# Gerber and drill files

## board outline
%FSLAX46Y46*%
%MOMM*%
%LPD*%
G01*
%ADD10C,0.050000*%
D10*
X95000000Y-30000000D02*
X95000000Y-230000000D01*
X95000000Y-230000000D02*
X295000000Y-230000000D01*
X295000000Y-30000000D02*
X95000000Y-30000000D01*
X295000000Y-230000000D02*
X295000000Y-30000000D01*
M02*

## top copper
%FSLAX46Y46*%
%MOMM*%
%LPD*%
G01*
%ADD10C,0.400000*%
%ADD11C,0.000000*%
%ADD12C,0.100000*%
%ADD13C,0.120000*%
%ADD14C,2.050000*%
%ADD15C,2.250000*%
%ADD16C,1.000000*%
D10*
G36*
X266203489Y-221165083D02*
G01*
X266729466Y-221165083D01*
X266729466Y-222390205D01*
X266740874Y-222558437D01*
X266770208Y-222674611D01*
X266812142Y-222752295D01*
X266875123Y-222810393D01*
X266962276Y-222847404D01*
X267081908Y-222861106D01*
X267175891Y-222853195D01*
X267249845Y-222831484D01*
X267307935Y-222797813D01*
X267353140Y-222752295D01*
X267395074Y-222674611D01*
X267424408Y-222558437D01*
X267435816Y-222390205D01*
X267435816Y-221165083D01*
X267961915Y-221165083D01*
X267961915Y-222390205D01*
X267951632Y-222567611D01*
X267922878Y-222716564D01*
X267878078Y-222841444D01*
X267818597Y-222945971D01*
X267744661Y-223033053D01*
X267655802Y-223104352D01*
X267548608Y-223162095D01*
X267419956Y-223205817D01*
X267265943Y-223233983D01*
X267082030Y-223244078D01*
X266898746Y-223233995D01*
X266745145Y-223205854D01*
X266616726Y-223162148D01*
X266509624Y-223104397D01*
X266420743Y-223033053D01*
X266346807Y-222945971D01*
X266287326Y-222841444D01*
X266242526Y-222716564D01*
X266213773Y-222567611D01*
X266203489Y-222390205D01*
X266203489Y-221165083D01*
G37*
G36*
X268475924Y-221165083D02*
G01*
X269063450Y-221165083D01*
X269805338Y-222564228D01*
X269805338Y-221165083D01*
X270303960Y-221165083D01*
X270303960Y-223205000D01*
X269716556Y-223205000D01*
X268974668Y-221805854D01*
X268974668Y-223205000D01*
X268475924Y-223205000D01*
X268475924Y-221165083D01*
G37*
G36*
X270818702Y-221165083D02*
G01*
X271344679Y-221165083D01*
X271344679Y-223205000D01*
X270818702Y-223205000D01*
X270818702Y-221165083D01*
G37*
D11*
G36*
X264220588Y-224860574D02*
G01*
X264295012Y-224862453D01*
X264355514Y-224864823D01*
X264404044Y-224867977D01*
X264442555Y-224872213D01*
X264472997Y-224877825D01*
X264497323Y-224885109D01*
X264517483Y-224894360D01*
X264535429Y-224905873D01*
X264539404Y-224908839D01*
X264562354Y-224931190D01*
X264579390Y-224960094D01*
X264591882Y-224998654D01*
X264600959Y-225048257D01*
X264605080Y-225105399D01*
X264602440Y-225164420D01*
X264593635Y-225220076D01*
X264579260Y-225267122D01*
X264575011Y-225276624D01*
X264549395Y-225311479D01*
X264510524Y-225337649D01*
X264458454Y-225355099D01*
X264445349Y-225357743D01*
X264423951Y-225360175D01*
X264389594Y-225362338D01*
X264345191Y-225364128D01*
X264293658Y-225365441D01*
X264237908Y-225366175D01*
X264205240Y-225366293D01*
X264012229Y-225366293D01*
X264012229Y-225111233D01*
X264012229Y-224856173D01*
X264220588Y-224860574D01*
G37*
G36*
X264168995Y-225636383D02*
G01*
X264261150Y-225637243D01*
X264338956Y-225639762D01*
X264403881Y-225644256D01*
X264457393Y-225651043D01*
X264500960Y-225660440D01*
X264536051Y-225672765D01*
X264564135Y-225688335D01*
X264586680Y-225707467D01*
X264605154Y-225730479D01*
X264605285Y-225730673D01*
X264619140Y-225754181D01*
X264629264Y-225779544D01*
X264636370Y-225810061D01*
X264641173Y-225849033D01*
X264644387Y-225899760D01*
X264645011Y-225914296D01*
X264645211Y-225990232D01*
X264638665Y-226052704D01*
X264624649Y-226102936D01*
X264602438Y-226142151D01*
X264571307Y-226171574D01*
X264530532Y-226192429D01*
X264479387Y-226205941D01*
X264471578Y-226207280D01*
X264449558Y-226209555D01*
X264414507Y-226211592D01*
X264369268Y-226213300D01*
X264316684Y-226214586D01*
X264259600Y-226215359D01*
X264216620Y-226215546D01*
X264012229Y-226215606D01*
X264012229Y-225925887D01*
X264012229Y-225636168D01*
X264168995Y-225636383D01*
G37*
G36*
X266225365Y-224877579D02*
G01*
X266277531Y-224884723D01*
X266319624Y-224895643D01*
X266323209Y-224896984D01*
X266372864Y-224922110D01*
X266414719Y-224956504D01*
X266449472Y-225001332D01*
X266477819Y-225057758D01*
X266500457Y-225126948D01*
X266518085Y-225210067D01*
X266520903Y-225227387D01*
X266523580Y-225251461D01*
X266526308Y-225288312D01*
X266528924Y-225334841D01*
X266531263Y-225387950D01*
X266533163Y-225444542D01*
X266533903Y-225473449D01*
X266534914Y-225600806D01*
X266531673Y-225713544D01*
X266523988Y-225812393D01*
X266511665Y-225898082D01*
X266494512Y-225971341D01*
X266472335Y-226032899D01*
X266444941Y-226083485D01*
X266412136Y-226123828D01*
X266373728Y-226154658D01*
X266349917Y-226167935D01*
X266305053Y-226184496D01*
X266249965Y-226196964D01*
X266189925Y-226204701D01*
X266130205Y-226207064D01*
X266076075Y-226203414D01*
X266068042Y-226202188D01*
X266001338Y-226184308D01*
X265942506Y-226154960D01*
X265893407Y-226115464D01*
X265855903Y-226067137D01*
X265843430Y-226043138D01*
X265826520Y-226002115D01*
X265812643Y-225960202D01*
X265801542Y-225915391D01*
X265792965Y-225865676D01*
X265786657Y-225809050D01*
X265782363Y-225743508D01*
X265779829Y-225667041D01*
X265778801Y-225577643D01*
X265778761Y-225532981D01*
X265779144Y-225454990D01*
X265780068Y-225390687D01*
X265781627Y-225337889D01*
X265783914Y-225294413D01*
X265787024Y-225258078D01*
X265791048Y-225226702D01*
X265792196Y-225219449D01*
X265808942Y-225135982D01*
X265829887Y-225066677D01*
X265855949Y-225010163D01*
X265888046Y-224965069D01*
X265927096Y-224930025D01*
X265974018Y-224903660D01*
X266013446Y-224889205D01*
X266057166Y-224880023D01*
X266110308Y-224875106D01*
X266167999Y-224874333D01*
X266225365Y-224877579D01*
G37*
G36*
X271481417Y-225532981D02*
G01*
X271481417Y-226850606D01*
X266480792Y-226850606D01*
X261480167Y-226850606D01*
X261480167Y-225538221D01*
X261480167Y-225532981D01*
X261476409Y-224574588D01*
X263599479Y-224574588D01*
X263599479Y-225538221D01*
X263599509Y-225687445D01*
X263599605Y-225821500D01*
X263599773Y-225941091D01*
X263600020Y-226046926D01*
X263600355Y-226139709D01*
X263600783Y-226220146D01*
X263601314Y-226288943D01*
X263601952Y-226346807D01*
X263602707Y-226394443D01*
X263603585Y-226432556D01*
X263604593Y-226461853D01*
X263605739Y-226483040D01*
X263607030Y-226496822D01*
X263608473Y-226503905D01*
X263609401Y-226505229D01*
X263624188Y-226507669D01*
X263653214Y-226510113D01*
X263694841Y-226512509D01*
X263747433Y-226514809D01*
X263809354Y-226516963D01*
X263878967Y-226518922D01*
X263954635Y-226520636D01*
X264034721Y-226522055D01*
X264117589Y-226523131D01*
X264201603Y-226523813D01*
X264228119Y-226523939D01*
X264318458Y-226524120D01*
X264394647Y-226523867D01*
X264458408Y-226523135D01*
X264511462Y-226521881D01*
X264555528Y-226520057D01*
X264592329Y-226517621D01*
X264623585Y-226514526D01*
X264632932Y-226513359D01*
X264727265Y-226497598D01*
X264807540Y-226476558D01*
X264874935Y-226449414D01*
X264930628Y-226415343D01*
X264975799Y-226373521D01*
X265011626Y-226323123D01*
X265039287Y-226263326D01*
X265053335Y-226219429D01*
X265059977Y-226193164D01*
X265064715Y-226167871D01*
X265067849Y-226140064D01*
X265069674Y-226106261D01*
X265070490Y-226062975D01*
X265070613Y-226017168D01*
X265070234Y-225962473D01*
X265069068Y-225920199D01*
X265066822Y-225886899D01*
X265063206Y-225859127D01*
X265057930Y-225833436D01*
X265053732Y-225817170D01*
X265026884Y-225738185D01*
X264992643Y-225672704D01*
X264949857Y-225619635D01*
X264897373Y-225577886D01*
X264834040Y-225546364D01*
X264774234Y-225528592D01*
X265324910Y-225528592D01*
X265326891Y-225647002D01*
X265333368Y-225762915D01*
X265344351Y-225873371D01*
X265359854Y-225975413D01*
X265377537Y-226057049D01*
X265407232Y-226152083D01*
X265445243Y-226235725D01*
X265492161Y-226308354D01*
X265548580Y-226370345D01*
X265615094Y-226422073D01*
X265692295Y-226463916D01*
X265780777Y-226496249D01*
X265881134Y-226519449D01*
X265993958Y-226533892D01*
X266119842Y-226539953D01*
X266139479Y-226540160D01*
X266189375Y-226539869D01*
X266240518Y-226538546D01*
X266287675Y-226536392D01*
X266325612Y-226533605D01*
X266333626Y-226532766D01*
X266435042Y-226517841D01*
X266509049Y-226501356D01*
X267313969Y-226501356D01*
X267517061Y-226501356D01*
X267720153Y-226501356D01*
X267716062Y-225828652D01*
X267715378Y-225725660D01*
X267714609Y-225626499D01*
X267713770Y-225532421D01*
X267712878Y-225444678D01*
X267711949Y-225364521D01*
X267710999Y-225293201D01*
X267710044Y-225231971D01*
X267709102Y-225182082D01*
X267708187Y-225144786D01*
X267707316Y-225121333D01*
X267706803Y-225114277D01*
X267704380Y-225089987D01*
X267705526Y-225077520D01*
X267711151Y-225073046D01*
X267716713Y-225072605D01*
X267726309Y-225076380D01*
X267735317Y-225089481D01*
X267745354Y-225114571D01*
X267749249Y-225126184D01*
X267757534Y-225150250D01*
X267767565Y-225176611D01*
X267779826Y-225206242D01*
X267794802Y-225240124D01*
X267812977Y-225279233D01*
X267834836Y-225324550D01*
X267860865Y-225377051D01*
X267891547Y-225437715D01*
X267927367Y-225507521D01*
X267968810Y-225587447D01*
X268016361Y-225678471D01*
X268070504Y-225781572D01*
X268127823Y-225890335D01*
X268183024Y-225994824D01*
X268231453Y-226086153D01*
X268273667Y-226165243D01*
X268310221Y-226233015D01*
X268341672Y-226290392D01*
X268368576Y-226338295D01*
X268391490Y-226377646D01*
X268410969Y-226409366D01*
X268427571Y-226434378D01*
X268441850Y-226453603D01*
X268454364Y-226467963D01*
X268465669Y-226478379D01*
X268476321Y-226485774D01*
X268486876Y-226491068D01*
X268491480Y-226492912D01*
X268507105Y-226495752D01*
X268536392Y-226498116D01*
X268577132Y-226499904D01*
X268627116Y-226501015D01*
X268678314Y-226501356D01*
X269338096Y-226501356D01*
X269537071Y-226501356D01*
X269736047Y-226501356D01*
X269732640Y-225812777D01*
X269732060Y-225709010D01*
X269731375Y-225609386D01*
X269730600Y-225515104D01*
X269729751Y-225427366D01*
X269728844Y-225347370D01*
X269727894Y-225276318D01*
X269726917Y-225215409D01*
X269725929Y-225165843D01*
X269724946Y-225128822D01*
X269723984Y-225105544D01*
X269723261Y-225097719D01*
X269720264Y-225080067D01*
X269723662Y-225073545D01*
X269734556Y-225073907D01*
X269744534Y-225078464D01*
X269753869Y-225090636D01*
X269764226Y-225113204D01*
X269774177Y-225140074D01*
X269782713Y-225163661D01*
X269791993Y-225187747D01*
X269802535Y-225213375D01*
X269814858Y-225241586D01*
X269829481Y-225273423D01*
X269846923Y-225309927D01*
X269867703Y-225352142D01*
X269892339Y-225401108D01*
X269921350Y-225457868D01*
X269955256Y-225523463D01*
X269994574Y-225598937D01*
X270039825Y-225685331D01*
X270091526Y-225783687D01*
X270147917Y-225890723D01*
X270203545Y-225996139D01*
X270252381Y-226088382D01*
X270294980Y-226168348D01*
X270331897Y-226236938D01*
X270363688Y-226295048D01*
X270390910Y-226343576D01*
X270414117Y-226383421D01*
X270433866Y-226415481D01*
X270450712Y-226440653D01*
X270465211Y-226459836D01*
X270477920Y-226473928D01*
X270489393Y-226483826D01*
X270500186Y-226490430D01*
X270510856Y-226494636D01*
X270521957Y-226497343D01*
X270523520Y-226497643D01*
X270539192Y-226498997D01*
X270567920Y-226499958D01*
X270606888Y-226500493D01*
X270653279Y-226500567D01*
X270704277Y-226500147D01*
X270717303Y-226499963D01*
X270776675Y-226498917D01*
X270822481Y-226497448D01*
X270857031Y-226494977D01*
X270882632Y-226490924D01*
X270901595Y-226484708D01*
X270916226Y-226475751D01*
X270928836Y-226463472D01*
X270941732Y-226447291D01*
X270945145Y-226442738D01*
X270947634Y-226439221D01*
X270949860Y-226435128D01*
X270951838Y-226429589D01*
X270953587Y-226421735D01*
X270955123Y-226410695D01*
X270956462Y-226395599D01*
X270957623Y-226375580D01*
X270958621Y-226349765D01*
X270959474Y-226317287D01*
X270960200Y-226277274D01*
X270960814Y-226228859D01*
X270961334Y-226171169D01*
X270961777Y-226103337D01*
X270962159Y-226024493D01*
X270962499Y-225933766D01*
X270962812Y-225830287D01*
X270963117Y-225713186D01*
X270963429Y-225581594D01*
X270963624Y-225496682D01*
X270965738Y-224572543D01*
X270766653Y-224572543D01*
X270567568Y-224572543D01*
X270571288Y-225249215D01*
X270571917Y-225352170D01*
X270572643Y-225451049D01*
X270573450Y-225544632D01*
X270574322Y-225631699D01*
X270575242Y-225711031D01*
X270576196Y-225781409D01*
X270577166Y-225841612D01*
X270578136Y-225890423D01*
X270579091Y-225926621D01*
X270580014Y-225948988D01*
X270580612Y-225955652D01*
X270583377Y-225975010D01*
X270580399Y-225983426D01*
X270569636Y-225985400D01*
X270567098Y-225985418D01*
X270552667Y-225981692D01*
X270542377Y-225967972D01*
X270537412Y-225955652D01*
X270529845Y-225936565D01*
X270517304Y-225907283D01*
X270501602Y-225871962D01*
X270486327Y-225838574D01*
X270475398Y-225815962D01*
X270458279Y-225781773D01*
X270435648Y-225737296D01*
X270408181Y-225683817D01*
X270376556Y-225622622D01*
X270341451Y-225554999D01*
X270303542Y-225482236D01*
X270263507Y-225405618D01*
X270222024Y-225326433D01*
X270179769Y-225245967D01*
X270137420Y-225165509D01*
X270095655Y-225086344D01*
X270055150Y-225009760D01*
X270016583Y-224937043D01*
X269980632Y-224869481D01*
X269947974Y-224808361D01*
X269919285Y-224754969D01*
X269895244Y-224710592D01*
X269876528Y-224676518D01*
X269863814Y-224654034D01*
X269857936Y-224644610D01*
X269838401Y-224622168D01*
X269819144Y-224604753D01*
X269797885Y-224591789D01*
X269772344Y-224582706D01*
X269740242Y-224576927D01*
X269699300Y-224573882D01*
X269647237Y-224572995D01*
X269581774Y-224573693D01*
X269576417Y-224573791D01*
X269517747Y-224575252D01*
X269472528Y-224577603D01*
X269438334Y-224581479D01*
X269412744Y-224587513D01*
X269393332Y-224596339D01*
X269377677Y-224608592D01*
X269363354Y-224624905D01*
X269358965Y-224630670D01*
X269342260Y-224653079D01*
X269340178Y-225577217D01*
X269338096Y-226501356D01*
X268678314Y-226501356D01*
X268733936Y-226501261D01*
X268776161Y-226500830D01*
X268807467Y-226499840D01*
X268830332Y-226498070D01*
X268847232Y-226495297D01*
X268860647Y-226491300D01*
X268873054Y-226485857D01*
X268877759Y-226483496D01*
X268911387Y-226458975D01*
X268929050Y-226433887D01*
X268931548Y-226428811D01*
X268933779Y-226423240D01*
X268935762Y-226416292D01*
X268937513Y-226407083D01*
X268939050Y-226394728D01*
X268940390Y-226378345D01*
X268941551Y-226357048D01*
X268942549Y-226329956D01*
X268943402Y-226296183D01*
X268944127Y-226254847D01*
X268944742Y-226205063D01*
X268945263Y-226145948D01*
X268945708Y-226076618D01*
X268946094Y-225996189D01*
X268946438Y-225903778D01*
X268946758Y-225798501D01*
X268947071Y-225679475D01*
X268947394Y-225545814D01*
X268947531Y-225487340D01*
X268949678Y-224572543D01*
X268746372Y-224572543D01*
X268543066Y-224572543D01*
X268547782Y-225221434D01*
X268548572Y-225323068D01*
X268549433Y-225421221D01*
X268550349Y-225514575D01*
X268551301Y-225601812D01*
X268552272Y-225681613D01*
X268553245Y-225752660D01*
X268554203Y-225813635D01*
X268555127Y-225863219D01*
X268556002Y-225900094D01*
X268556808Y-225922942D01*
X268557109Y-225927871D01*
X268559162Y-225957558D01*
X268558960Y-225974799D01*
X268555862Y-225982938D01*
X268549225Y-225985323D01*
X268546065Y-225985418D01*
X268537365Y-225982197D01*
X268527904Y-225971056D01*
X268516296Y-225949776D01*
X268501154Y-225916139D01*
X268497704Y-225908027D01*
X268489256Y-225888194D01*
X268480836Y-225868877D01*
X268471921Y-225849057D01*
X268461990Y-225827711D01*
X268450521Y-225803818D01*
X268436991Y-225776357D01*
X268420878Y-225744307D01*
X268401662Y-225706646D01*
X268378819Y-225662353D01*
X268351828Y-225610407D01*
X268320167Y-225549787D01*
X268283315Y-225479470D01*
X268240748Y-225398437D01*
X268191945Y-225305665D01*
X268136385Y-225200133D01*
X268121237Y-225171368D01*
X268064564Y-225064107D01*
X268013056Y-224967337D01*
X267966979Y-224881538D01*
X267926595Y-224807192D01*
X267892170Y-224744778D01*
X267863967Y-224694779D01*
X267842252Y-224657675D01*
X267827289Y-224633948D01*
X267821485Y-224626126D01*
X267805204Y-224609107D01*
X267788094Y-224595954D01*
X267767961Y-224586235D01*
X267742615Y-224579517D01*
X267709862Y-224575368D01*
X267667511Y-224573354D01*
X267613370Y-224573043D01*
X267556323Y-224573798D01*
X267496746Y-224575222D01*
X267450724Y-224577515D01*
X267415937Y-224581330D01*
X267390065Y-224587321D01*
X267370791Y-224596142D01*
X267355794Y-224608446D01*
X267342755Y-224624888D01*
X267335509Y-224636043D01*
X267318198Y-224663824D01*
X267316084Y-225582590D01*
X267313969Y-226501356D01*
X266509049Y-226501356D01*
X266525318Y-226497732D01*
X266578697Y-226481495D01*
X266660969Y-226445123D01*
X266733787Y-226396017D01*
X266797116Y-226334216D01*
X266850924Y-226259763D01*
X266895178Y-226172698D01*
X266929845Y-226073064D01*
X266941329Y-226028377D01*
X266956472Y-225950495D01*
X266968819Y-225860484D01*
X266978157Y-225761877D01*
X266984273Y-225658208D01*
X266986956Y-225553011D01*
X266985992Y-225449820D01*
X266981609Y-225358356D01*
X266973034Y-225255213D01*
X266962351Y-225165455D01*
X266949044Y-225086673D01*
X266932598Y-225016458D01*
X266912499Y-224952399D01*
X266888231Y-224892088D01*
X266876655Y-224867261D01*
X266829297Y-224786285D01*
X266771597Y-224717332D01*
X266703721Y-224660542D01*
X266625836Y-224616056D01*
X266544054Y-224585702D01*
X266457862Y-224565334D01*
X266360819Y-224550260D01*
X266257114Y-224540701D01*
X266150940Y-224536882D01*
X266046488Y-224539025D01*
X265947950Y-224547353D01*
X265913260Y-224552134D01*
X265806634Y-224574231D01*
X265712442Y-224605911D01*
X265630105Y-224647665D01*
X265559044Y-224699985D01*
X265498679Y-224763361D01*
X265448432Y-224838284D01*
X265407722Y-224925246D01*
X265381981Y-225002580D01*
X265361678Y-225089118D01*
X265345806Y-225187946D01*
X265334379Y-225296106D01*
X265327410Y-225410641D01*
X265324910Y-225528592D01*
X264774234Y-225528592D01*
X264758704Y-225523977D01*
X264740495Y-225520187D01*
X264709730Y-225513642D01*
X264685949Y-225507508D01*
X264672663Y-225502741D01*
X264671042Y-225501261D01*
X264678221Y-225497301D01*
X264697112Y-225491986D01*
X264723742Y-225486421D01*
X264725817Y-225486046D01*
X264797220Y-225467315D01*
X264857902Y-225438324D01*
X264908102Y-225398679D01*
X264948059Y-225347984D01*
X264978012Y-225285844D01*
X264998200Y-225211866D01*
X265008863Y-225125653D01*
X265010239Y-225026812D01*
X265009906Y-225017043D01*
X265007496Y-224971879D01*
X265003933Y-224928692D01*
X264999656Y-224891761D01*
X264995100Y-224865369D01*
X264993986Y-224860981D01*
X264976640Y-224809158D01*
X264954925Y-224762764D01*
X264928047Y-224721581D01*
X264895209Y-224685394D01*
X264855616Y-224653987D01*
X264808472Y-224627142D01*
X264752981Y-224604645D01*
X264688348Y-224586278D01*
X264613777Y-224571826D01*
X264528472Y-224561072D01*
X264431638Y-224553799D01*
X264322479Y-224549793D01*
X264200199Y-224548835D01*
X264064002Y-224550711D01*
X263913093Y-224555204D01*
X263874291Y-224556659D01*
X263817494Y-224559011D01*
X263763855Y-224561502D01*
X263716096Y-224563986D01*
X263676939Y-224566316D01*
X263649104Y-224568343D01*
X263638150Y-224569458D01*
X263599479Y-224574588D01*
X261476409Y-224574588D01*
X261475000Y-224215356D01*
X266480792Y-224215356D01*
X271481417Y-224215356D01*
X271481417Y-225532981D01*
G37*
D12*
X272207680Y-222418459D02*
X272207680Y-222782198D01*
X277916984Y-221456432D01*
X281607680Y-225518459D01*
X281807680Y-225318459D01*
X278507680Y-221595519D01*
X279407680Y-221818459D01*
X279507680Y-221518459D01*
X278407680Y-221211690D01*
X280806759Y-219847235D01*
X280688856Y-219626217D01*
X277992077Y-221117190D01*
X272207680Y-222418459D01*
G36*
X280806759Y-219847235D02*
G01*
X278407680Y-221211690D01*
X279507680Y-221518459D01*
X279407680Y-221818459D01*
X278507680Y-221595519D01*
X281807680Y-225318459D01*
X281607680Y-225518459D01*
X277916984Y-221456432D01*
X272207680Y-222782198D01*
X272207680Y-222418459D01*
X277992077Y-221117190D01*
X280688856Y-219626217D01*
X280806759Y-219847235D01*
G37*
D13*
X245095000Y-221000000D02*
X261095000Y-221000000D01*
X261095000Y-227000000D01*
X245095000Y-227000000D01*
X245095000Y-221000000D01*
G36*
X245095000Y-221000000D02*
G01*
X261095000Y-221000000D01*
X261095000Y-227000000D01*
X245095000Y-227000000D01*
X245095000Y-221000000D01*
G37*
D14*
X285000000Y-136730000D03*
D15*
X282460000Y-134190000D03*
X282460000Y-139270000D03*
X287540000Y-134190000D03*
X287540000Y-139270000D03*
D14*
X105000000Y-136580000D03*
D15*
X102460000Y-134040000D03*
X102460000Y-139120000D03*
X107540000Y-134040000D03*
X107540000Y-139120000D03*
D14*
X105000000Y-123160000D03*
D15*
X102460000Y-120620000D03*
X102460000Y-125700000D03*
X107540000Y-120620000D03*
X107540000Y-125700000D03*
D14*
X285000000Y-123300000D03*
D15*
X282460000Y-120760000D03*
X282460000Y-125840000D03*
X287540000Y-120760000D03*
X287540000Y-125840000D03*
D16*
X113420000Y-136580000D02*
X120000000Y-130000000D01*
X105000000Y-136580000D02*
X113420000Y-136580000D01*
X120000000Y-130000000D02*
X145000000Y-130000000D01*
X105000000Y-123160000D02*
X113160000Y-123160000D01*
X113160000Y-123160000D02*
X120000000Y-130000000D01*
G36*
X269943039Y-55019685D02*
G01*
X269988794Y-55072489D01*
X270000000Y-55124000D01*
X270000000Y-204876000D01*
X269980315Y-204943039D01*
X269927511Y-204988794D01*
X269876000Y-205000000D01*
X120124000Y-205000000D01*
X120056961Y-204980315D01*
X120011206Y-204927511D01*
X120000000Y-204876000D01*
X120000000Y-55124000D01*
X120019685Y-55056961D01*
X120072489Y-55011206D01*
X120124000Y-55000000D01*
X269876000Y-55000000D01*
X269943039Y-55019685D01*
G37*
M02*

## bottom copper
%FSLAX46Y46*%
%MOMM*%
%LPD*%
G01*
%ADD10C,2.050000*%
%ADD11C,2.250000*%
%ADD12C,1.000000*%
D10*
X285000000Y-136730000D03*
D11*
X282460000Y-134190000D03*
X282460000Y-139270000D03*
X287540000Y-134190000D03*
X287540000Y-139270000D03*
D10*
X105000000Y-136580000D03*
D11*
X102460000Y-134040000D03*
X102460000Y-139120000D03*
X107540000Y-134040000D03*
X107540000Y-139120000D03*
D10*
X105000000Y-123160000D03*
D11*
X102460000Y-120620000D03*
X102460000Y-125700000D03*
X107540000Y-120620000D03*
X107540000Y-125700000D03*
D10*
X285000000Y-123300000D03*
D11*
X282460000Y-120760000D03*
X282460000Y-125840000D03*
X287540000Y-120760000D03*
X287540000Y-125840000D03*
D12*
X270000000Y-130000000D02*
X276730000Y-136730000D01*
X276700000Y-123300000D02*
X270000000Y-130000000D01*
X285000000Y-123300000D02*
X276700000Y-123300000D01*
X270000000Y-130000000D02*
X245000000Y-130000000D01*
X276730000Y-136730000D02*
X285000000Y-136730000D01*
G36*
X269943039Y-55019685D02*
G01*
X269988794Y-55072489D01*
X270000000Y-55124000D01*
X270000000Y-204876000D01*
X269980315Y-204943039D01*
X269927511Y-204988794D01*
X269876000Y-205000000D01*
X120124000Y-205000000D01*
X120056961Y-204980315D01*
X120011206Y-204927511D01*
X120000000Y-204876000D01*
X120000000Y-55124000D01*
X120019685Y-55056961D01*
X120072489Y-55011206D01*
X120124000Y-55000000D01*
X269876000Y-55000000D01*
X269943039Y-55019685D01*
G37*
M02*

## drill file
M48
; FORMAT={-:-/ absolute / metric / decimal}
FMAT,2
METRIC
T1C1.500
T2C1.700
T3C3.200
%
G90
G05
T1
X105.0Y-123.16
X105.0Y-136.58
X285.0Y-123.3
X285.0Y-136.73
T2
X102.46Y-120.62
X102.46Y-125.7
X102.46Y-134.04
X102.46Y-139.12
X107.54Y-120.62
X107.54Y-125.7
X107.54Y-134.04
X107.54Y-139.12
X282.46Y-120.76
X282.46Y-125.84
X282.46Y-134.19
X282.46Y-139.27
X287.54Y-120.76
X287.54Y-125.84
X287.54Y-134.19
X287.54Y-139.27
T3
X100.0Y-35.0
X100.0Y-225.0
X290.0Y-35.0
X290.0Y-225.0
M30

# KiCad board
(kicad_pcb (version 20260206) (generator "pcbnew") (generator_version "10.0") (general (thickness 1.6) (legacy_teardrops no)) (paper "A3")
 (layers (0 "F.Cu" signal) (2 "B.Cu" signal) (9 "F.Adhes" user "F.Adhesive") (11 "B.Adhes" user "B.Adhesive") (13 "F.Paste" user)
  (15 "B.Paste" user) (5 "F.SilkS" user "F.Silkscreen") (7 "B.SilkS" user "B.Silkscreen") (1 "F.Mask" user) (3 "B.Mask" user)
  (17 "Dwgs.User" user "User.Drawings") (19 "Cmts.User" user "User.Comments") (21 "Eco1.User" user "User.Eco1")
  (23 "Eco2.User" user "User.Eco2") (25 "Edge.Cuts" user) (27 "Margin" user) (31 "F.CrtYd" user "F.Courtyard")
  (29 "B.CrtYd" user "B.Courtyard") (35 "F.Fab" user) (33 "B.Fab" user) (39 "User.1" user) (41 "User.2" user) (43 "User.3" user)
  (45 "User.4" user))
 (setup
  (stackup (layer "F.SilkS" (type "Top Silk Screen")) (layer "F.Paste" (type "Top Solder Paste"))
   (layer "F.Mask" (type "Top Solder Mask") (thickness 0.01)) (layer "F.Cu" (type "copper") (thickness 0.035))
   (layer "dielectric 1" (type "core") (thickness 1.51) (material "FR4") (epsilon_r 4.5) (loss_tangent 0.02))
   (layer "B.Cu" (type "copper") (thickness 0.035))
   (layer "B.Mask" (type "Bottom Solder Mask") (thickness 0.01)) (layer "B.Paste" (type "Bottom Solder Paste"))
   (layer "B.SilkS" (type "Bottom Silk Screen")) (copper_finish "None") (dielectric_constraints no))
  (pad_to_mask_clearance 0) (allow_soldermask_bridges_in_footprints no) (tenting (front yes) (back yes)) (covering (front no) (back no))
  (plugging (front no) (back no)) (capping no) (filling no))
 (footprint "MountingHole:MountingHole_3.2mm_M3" (layer "F.Cu") (at 290 35)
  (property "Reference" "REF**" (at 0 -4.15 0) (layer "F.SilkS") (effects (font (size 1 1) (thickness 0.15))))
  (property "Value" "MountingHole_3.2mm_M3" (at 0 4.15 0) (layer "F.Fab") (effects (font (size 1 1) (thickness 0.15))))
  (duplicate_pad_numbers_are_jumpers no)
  (pad "" np_thru_hole circle (at 0 0) (size 3.2 3.2) (drill 3.2) (layers "*.Cu" "*.Mask")))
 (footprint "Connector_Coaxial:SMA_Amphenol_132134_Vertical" (layer "F.Cu") (at 285 136.73)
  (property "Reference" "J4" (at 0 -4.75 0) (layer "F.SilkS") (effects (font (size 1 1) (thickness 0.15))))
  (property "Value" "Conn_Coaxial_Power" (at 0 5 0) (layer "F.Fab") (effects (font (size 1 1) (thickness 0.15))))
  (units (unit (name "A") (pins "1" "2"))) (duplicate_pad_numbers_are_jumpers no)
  (pad "1" thru_hole circle (at 0 0) (size 2.05 2.05) (drill 1.5) (layers "*.Cu" "*.Mask") (remove_unused_layers no) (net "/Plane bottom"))
  (pad "2" thru_hole circle (at -2.54 -2.54) (size 2.25 2.25) (drill 1.7) (layers "*.Cu" "*.Mask") (remove_unused_layers no) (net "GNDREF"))
  (pad "2" thru_hole circle (at -2.54 2.54) (size 2.25 2.25) (drill 1.7) (layers "*.Cu" "*.Mask") (remove_unused_layers no) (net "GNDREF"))
  (pad "2" thru_hole circle (at 2.54 -2.54) (size 2.25 2.25) (drill 1.7) (layers "*.Cu" "*.Mask") (remove_unused_layers no) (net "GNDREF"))
  (pad "2" thru_hole circle (at 2.54 2.54) (size 2.25 2.25) (drill 1.7) (layers "*.Cu" "*.Mask") (remove_unused_layers no) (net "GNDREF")))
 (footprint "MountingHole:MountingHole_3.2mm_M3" (layer "F.Cu") (at 100 35)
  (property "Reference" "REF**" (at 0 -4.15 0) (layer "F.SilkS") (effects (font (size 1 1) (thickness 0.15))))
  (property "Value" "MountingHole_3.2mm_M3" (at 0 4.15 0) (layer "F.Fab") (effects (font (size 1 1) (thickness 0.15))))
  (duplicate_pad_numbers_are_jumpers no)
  (pad "" np_thru_hole circle (at 0 0) (size 3.2 3.2) (drill 3.2) (layers "*.Cu" "*.Mask")))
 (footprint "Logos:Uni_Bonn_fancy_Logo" (layer "F.Cu") (at 266.5 222)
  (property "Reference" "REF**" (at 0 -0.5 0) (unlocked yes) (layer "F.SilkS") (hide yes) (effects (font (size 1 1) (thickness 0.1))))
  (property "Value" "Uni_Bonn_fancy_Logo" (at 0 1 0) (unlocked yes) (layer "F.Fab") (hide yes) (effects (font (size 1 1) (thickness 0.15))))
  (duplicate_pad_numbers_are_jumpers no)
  (fp_poly
   (pts (xy -2.279412 2.860574) (xy -2.204988 2.862453) (xy -2.144486 2.864823) (xy -2.095956 2.867977) (xy -2.057445 2.872213)
    (xy -2.027003 2.877825) (xy -2.002677 2.885109) (xy -1.982517 2.89436) (xy -1.964571 2.905873) (xy -1.960596 2.908839)
    (xy -1.937646 2.93119) (xy -1.92061 2.960094) (xy -1.908118 2.998654) (xy -1.899041 3.048257) (xy -1.89492 3.105399)
    (xy -1.89756 3.16442) (xy -1.906365 3.220076) (xy -1.92074 3.267122) (xy -1.924989 3.276624) (xy -1.950605 3.311479)
    (xy -1.989476 3.337649) (xy -2.041546 3.355099) (xy -2.054651 3.357743) (xy -2.076049 3.360175) (xy -2.110406 3.362338)
    (xy -2.154809 3.364128) (xy -2.206342 3.365441) (xy -2.262092 3.366175) (xy -2.29476 3.366293) (xy -2.487771 3.366293)
    (xy -2.487771 3.111233) (xy -2.487771 2.856173))
   (stroke (width 0) (type solid)) (fill yes) (layer "F.Cu"))
  (fp_poly
   (pts (xy -2.331005 3.636383) (xy -2.23885 3.637243) (xy -2.161044 3.639762) (xy -2.096119 3.644256) (xy -2.042607 3.651043)
    (xy -1.99904 3.66044) (xy -1.963949 3.672765) (xy -1.935865 3.688335) (xy -1.91332 3.707467) (xy -1.894846 3.730479)
    (xy -1.894715 3.730673) (xy -1.88086 3.754181) (xy -1.870736 3.779544) (xy -1.86363 3.810061) (xy -1.858827 3.849033)
    (xy -1.855613 3.89976) (xy -1.854989 3.914296) (xy -1.854789 3.990232) (xy -1.861335 4.052704) (xy -1.875351 4.102936)
    (xy -1.897562 4.142151) (xy -1.928693 4.171574) (xy -1.969468 4.192429) (xy -2.020613 4.205941) (xy -2.028422 4.20728)
    (xy -2.050442 4.209555) (xy -2.085493 4.211592) (xy -2.130732 4.2133) (xy -2.183316 4.214586) (xy -2.2404 4.215359)
    (xy -2.28338 4.215546) (xy -2.487771 4.215606) (xy -2.487771 3.925887) (xy -2.487771 3.636168))
   (stroke (width 0) (type solid)) (fill yes) (layer "F.Cu"))
  (fp_poly
   (pts (xy -0.274635 2.877579) (xy -0.222469 2.884723) (xy -0.180376 2.895643) (xy -0.176791 2.896984) (xy -0.127136 2.92211)
    (xy -0.085281 2.956504) (xy -0.050528 3.001332) (xy -0.022181 3.057758) (xy 0.000457 3.126948) (xy 0.018085 3.210067)
    (xy 0.020903 3.227387) (xy 0.02358 3.251461) (xy 0.026308 3.288312) (xy 0.028924 3.334841) (xy 0.031263 3.38795) (xy 0.033163 3.444542)
    (xy 0.033903 3.473449) (xy 0.034914 3.600806) (xy 0.031673 3.713544) (xy 0.023988 3.812393) (xy 0.011665 3.898082)
    (xy -0.005488 3.971341) (xy -0.027665 4.032899) (xy -0.055059 4.083485) (xy -0.087864 4.123828) (xy -0.126272 4.154658)
    (xy -0.150083 4.167935) (xy -0.194947 4.184496) (xy -0.250035 4.196964) (xy -0.310075 4.204701) (xy -0.369795 4.207064)
    (xy -0.423925 4.203414) (xy -0.431958 4.202188) (xy -0.498662 4.184308) (xy -0.557494 4.15496) (xy -0.606593 4.115464)
    (xy -0.644097 4.067137) (xy -0.65657 4.043138) (xy -0.67348 4.002115) (xy -0.687357 3.960202) (xy -0.698458 3.915391)
    (xy -0.707035 3.865676) (xy -0.713343 3.80905) (xy -0.717637 3.743508) (xy -0.720171 3.667041) (xy -0.721199 3.577643)
    (xy -0.721239 3.532981) (xy -0.720856 3.45499) (xy -0.719932 3.390687) (xy -0.718373 3.337889) (xy -0.716086 3.294413)
    (xy -0.712976 3.258078) (xy -0.708952 3.226702) (xy -0.707804 3.219449) (xy -0.691058 3.135982) (xy -0.670113 3.066677)
    (xy -0.644051 3.010163) (xy -0.611954 2.965069) (xy -0.572904 2.930025) (xy -0.525982 2.90366) (xy -0.486554 2.889205)
    (xy -0.442834 2.880023) (xy -0.389692 2.875106) (xy -0.332001 2.874333))
   (stroke (width 0) (type solid)) (fill yes) (layer "F.Cu"))
  (fp_poly
   (pts (xy 4.981417 3.532981) (xy 4.981417 4.850606) (xy -0.019208 4.850606) (xy -5.019833 4.850606) (xy -5.019833 3.538221)
    (xy -2.900521 3.538221) (xy -2.900491 3.687445) (xy -2.900395 3.8215) (xy -2.900227 3.941091) (xy -2.89998 4.046926)
    (xy -2.899645 4.139709) (xy -2.899217 4.220146) (xy -2.898686 4.288943) (xy -2.898048 4.346807) (xy -2.897293 4.394443)
    (xy -2.896415 4.432556) (xy -2.895407 4.461853) (xy -2.894261 4.48304) (xy -2.89297 4.496822) (xy -2.891527 4.503905)
    (xy -2.890599 4.505229) (xy -2.875812 4.507669) (xy -2.846786 4.510113) (xy -2.805159 4.512509) (xy -2.752567 4.514809)
    (xy -2.690646 4.516963) (xy -2.621033 4.518922) (xy -2.545365 4.520636) (xy -2.465279 4.522055) (xy -2.382411 4.523131)
    (xy -2.298397 4.523813) (xy -2.271881 4.523939) (xy -2.181542 4.52412) (xy -2.105353 4.523867) (xy -2.041592 4.523135)
    (xy -1.988538 4.521881) (xy -1.944472 4.520057) (xy -1.907671 4.517621) (xy -1.876415 4.514526) (xy -1.867068 4.513359)
    (xy -1.772735 4.497598) (xy -1.69246 4.476558) (xy -1.625065 4.449414) (xy -1.569372 4.415343) (xy -1.524201 4.373521)
    (xy -1.488374 4.323123) (xy -1.460713 4.263326) (xy -1.446665 4.219429) (xy -1.440023 4.193164) (xy -1.435285 4.167871)
    (xy -1.432151 4.140064) (xy -1.430326 4.106261) (xy -1.42951 4.062975) (xy -1.429387 4.017168) (xy -1.429766 3.962473)
    (xy -1.430932 3.920199) (xy -1.433178 3.886899) (xy -1.436794 3.859127) (xy -1.44207 3.833436) (xy -1.446268 3.81717)
    (xy -1.473116 3.738185) (xy -1.507357 3.672704) (xy -1.550143 3.619635) (xy -1.602627 3.577886) (xy -1.66596 3.546364)
    (xy -1.725766 3.528592) (xy -1.17509 3.528592) (xy -1.173109 3.647002) (xy -1.166632 3.762915) (xy -1.155649 3.873371)
    (xy -1.140146 3.975413) (xy -1.122463 4.057049) (xy -1.092768 4.152083) (xy -1.054757 4.235725) (xy -1.007839 4.308354)
    (xy -0.95142 4.370345) (xy -0.884906 4.422073) (xy -0.807705 4.463916) (xy -0.719223 4.496249) (xy -0.618866 4.519449)
    (xy -0.506042 4.533892) (xy -0.380158 4.539953) (xy -0.360521 4.54016) (xy -0.310625 4.539869) (xy -0.259482 4.538546)
    (xy -0.212325 4.536392) (xy -0.174388 4.533605) (xy -0.166374 4.532766) (xy -0.064958 4.517841) (xy 0.009049 4.501356)
    (xy 0.813969 4.501356) (xy 1.017061 4.501356) (xy 1.220153 4.501356) (xy 1.216062 3.828652) (xy 1.215378 3.72566) (xy 1.214609 3.626499)
    (xy 1.21377 3.532421) (xy 1.212878 3.444678) (xy 1.211949 3.364521) (xy 1.210999 3.293201) (xy 1.210044 3.231971) (xy 1.209102 3.182082)
    (xy 1.208187 3.144786) (xy 1.207316 3.121333) (xy 1.206803 3.114277) (xy 1.20438 3.089987) (xy 1.205526 3.07752) (xy 1.211151 3.073046)
    (xy 1.216713 3.072605) (xy 1.226309 3.07638) (xy 1.235317 3.089481) (xy 1.245354 3.114571) (xy 1.249249 3.126184) (xy 1.257534 3.15025)
    (xy 1.267565 3.176611) (xy 1.279826 3.206242) (xy 1.294802 3.240124) (xy 1.312977 3.279233) (xy 1.334836 3.32455) (xy 1.360865 3.377051)
    (xy 1.391547 3.437715) (xy 1.427367 3.507521) (xy 1.46881 3.587447) (xy 1.516361 3.678471) (xy 1.570504 3.781572) (xy 1.627823 3.890335)
    (xy 1.683024 3.994824) (xy 1.731453 4.086153) (xy 1.773667 4.165243) (xy 1.810221 4.233015) (xy 1.841672 4.290392)
    (xy 1.868576 4.338295) (xy 1.89149 4.377646) (xy 1.910969 4.409366) (xy 1.927571 4.434378) (xy 1.94185 4.453603) (xy 1.954364 4.467963)
    (xy 1.965669 4.478379) (xy 1.976321 4.485774) (xy 1.986876 4.491068) (xy 1.99148 4.492912) (xy 2.007105 4.495752) (xy 2.036392 4.498116)
    (xy 2.077132 4.499904) (xy 2.127116 4.501015) (xy 2.178314 4.501356) (xy 2.838096 4.501356) (xy 3.037071 4.501356)
    (xy 3.236047 4.501356) (xy 3.23264 3.812777) (xy 3.23206 3.70901) (xy 3.231375 3.609386) (xy 3.2306 3.515104) (xy 3.229751 3.427366)
    (xy 3.228844 3.34737) (xy 3.227894 3.276318) (xy 3.226917 3.215409) (xy 3.225929 3.165843) (xy 3.224946 3.128822) (xy 3.223984 3.105544)
    (xy 3.223261 3.097719) (xy 3.220264 3.080067) (xy 3.223662 3.073545) (xy 3.234556 3.073907) (xy 3.244534 3.078464)
    (xy 3.253869 3.090636) (xy 3.264226 3.113204) (xy 3.274177 3.140074) (xy 3.282713 3.163661) (xy 3.291993 3.187747)
    (xy 3.302535 3.213375) (xy 3.314858 3.241586) (xy 3.329481 3.273423) (xy 3.346923 3.309927) (xy 3.367703 3.352142)
    (xy 3.392339 3.401108) (xy 3.42135 3.457868) (xy 3.455256 3.523463) (xy 3.494574 3.598937) (xy 3.539825 3.685331) (xy 3.591526 3.783687)
    (xy 3.647917 3.890723) (xy 3.703545 3.996139) (xy 3.752381 4.088382) (xy 3.79498 4.168348) (xy 3.831897 4.236938) (xy 3.863688 4.295048)
    (xy 3.89091 4.343576) (xy 3.914117 4.383421) (xy 3.933866 4.415481) (xy 3.950712 4.440653) (xy 3.965211 4.459836) (xy 3.97792 4.473928)
    (xy 3.989393 4.483826) (xy 4.000186 4.49043) (xy 4.010856 4.494636) (xy 4.021957 4.497343) (xy 4.02352 4.497643) (xy 4.039192 4.498997)
    (xy 4.06792 4.499958) (xy 4.106888 4.500493) (xy 4.153279 4.500567) (xy 4.204277 4.500147) (xy 4.217303 4.499963) (xy 4.276675 4.498917)
    (xy 4.322481 4.497448) (xy 4.357031 4.494977) (xy 4.382632 4.490924) (xy 4.401595 4.484708) (xy 4.416226 4.475751)
    (xy 4.428836 4.463472) (xy 4.441732 4.447291) (xy 4.445145 4.442738) (xy 4.447634 4.439221) (xy 4.44986 4.435128) (xy 4.451838 4.429589)
    (xy 4.453587 4.421735) (xy 4.455123 4.410695) (xy 4.456462 4.395599) (xy 4.457623 4.37558) (xy 4.458621 4.349765) (xy 4.459474 4.317287)
    (xy 4.4602 4.277274) (xy 4.460814 4.228859) (xy 4.461334 4.171169) (xy 4.461777 4.103337) (xy 4.462159 4.024493) (xy 4.462499 3.933766)
    (xy 4.462812 3.830287) (xy 4.463117 3.713186) (xy 4.463429 3.581594) (xy 4.463624 3.496682) (xy 4.465738 2.572543)
    (xy 4.266653 2.572543) (xy 4.067568 2.572543) (xy 4.071288 3.249215) (xy 4.071917 3.35217) (xy 4.072643 3.451049) (xy 4.07345 3.544632)
    (xy 4.074322 3.631699) (xy 4.075242 3.711031) (xy 4.076196 3.781409) (xy 4.077166 3.841612) (xy 4.078136 3.890423)
    (xy 4.079091 3.926621) (xy 4.080014 3.948988) (xy 4.080612 3.955652) (xy 4.083377 3.97501) (xy 4.080399 3.983426) (xy 4.069636 3.9854)
    (xy 4.067098 3.985418) (xy 4.052667 3.981692) (xy 4.042377 3.967972) (xy 4.037412 3.955652) (xy 4.029845 3.936565)
    (xy 4.017304 3.907283) (xy 4.001602 3.871962) (xy 3.986327 3.838574) (xy 3.975398 3.815962) (xy 3.958279 3.781773)
    (xy 3.935648 3.737296) (xy 3.908181 3.683817) (xy 3.876556 3.622622) (xy 3.841451 3.554999) (xy 3.803542 3.482236)
    (xy 3.763507 3.405618) (xy 3.722024 3.326433) (xy 3.679769 3.245967) (xy 3.63742 3.165509) (xy 3.595655 3.086344) (xy 3.55515 3.00976)
    (xy 3.516583 2.937043) (xy 3.480632 2.869481) (xy 3.447974 2.808361) (xy 3.419285 2.754969) (xy 3.395244 2.710592)
    (xy 3.376528 2.676518) (xy 3.363814 2.654034) (xy 3.357936 2.64461) (xy 3.338401 2.622168) (xy 3.319144 2.604753) (xy 3.297885 2.591789)
    (xy 3.272344 2.582706) (xy 3.240242 2.576927) (xy 3.1993 2.573882) (xy 3.147237 2.572995) (xy 3.081774 2.573693) (xy 3.076417 2.573791)
    (xy 3.017747 2.575252) (xy 2.972528 2.577603) (xy 2.938334 2.581479) (xy 2.912744 2.587513) (xy 2.893332 2.596339)
    (xy 2.877677 2.608592) (xy 2.863354 2.624905) (xy 2.858965 2.63067) (xy 2.84226 2.653079) (xy 2.840178 3.577217) (xy 2.838096 4.501356)
    (xy 2.178314 4.501356) (xy 2.233936 4.501261) (xy 2.276161 4.50083) (xy 2.307467 4.49984) (xy 2.330332 4.49807) (xy 2.347232 4.495297)
    (xy 2.360647 4.4913) (xy 2.373054 4.485857) (xy 2.377759 4.483496) (xy 2.411387 4.458975) (xy 2.42905 4.433887) (xy 2.431548 4.428811)
    (xy 2.433779 4.42324) (xy 2.435762 4.416292) (xy 2.437513 4.407083) (xy 2.43905 4.394728) (xy 2.44039 4.378345) (xy 2.441551 4.357048)
    (xy 2.442549 4.329956) (xy 2.443402 4.296183) (xy 2.444127 4.254847) (xy 2.444742 4.205063) (xy 2.445263 4.145948)
    (xy 2.445708 4.076618) (xy 2.446094 3.996189) (xy 2.446438 3.903778) (xy 2.446758 3.798501) (xy 2.447071 3.679475)
    (xy 2.447394 3.545814) (xy 2.447531 3.48734) (xy 2.449678 2.572543) (xy 2.246372 2.572543) (xy 2.043066 2.572543) (xy 2.047782 3.221434)
    (xy 2.048572 3.323068) (xy 2.049433 3.421221) (xy 2.050349 3.514575) (xy 2.051301 3.601812) (xy 2.052272 3.681613) (xy 2.053245 3.75266)
    (xy 2.054203 3.813635) (xy 2.055127 3.863219) (xy 2.056002 3.900094) (xy 2.056808 3.922942) (xy 2.057109 3.927871)
    (xy 2.059162 3.957558) (xy 2.05896 3.974799) (xy 2.055862 3.982938) (xy 2.049225 3.985323) (xy 2.046065 3.985418) (xy 2.037365 3.982197)
    (xy 2.027904 3.971056) (xy 2.016296 3.949776) (xy 2.001154 3.916139) (xy 1.997704 3.908027) (xy 1.989256 3.888194)
    (xy 1.980836 3.868877) (xy 1.971921 3.849057) (xy 1.96199 3.827711) (xy 1.950521 3.803818) (xy 1.936991 3.776357) (xy 1.920878 3.744307)
    (xy 1.901662 3.706646) (xy 1.878819 3.662353) (xy 1.851828 3.610407) (xy 1.820167 3.549787) (xy 1.783315 3.47947) (xy 1.740748 3.398437)
    (xy 1.691945 3.305665) (xy 1.636385 3.200133) (xy 1.621237 3.171368) (xy 1.564564 3.064107) (xy 1.513056 2.967337)
    (xy 1.466979 2.881538) (xy 1.426595 2.807192) (xy 1.39217 2.744778) (xy 1.363967 2.694779) (xy 1.342252 2.657675) (xy 1.327289 2.633948)
    (xy 1.321485 2.626126) (xy 1.305204 2.609107) (xy 1.288094 2.595954) (xy 1.267961 2.586235) (xy 1.242615 2.579517)
    (xy 1.209862 2.575368) (xy 1.167511 2.573354) (xy 1.11337 2.573043) (xy 1.056323 2.573798) (xy 0.996746 2.575222) (xy 0.950724 2.577515)
    (xy 0.915937 2.58133) (xy 0.890065 2.587321) (xy 0.870791 2.596142) (xy 0.855794 2.608446) (xy 0.842755 2.624888) (xy 0.835509 2.636043)
    (xy 0.818198 2.663824) (xy 0.816084 3.58259) (xy 0.813969 4.501356) (xy 0.009049 4.501356) (xy 0.025318 4.497732) (xy 0.078697 4.481495)
    (xy 0.160969 4.445123) (xy 0.233787 4.396017) (xy 0.297116 4.334216) (xy 0.350924 4.259763) (xy 0.395178 4.172698)
    (xy 0.429845 4.073064) (xy 0.441329 4.028377) (xy 0.456472 3.950495) (xy 0.468819 3.860484) (xy 0.478157 3.761877)
    (xy 0.484273 3.658208) (xy 0.486956 3.553011) (xy 0.485992 3.44982) (xy 0.481609 3.358356) (xy 0.473034 3.255213) (xy 0.462351 3.165455)
    (xy 0.449044 3.086673) (xy 0.432598 3.016458) (xy 0.412499 2.952399) (xy 0.388231 2.892088) (xy 0.376655 2.867261)
    (xy 0.329297 2.786285) (xy 0.271597 2.717332) (xy 0.203721 2.660542) (xy 0.125836 2.616056) (xy 0.044054 2.585702)
    (xy -0.042138 2.565334) (xy -0.139181 2.55026) (xy -0.242886 2.540701) (xy -0.34906 2.536882) (xy -0.453512 2.539025)
    (xy -0.55205 2.547353) (xy -0.58674 2.552134) (xy -0.693366 2.574231) (xy -0.787558 2.605911) (xy -0.869895 2.647665)
    (xy -0.940956 2.699985) (xy -1.001321 2.763361) (xy -1.051568 2.838284) (xy -1.092278 2.925246) (xy -1.118019 3.00258)
    (xy -1.138322 3.089118) (xy -1.154194 3.187946) (xy -1.165621 3.296106) (xy -1.17259 3.410641) (xy -1.17509 3.528592)
    (xy -1.725766 3.528592) (xy -1.741296 3.523977) (xy -1.759505 3.520187) (xy -1.79027 3.513642) (xy -1.814051 3.507508)
    (xy -1.827337 3.502741) (xy -1.828958 3.501261) (xy -1.821779 3.497301) (xy -1.802888 3.491986) (xy -1.776258 3.486421)
    (xy -1.774183 3.486046) (xy -1.70278 3.467315) (xy -1.642098 3.438324) (xy -1.591898 3.398679) (xy -1.551941 3.347984)
    (xy -1.521988 3.285844) (xy -1.5018 3.211866) (xy -1.491137 3.125653) (xy -1.489761 3.026812) (xy -1.490094 3.017043)
    (xy -1.492504 2.971879) (xy -1.496067 2.928692) (xy -1.500344 2.891761) (xy -1.5049 2.865369) (xy -1.506014 2.860981)
    (xy -1.52336 2.809158) (xy -1.545075 2.762764) (xy -1.571953 2.721581) (xy -1.604791 2.685394) (xy -1.644384 2.653987)
    (xy -1.691528 2.627142) (xy -1.747019 2.604645) (xy -1.811652 2.586278) (xy -1.886223 2.571826) (xy -1.971528 2.561072)
    (xy -2.068362 2.553799) (xy -2.177521 2.549793) (xy -2.299801 2.548835) (xy -2.435998 2.550711) (xy -2.586907 2.555204)
    (xy -2.625709 2.556659) (xy -2.682506 2.559011) (xy -2.736145 2.561502) (xy -2.783904 2.563986) (xy -2.823061 2.566316)
    (xy -2.850896 2.568343) (xy -2.86185 2.569458) (xy -2.900521 2.574588) (xy -2.900521 3.538221) (xy -5.019833 3.538221)
    (xy -5.019833 3.532981) (xy -5.025 2.215356) (xy -0.019208 2.215356) (xy 4.981417 2.215356))
   (stroke (width 0) (type solid)) (fill yes) (layer "F.Cu"))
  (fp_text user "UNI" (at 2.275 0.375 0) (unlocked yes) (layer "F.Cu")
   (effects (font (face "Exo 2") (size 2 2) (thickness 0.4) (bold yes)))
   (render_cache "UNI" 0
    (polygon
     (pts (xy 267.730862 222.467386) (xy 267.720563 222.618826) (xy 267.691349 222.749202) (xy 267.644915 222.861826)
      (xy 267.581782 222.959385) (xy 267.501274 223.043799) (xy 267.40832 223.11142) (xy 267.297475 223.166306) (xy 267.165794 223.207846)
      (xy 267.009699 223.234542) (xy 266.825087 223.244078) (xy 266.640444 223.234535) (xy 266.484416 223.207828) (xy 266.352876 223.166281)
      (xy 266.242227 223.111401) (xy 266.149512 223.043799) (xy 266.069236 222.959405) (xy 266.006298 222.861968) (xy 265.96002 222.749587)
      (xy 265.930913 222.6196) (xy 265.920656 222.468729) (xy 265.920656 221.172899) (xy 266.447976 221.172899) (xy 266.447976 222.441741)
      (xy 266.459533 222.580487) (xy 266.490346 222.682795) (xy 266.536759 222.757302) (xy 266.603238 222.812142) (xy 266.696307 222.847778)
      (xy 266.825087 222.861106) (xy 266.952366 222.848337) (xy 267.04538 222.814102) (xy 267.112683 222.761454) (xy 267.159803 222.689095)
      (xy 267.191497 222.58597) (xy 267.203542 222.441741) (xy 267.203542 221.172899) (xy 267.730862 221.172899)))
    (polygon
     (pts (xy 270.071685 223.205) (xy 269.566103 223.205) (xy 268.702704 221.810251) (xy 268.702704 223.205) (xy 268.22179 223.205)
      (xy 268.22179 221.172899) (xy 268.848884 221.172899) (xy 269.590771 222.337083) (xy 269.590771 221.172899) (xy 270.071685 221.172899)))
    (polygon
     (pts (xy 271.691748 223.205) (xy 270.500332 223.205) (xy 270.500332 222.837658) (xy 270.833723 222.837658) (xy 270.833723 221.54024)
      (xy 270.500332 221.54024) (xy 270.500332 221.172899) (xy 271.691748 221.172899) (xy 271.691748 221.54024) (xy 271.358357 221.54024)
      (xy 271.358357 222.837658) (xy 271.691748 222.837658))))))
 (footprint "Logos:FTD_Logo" (layer "F.Cu") (at 277 222)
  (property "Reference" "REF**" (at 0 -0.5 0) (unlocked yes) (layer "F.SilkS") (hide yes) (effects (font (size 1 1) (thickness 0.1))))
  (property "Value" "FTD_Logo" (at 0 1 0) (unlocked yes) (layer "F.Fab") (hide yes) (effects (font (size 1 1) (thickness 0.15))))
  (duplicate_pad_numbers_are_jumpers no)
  (fp_poly
   (pts (xy -4.79232 0.418459) (xy -4.79232 0.782198) (xy 0.916984 -0.543568) (xy 4.60768 3.518459) (xy 4.80768 3.318459)
    (xy 1.50768 -0.404481) (xy 2.40768 -0.181541) (xy 2.50768 -0.481541) (xy 1.40768 -0.78831) (xy 3.806759 -2.152765)
    (xy 3.688856 -2.373783) (xy 0.992077 -0.88281))
   (stroke (width 0.1) (type solid)) (fill yes) (layer "F.Cu")))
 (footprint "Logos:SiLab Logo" (layer "F.Cu") (at 245.095 227)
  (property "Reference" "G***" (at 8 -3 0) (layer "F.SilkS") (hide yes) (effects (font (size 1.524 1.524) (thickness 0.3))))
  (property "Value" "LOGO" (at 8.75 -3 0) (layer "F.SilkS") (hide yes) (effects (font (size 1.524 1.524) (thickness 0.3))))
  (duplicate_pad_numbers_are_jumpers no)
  (fp_rect (start 0 -6) (end 16 0) (stroke (width 0.12) (type solid)) (fill yes) (layer "F.Cu")))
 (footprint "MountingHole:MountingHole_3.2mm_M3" (layer "F.Cu") (at 290 225)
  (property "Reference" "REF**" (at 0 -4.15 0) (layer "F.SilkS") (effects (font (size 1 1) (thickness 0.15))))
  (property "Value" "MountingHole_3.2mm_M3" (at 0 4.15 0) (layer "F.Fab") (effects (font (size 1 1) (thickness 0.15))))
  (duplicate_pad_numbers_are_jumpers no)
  (pad "" np_thru_hole circle (at 0 0) (size 3.2 3.2) (drill 3.2) (layers "*.Cu" "*.Mask")))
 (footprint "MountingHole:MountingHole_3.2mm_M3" (layer "F.Cu") (at 100 225)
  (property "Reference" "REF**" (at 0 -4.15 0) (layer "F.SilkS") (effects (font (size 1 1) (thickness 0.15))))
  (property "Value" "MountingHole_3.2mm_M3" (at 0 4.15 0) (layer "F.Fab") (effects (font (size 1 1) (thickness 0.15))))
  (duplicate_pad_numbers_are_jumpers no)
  (pad "" np_thru_hole circle (at 0 0) (size 3.2 3.2) (drill 3.2) (layers "*.Cu" "*.Mask")))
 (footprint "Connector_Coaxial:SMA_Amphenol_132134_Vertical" (layer "F.Cu") (at 105 136.58)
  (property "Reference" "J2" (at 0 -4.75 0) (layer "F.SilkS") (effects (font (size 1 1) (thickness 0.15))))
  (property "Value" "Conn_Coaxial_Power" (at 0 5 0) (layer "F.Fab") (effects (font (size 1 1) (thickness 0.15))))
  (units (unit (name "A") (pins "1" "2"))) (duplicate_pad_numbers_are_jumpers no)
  (pad "1" thru_hole circle (at 0 0) (size 2.05 2.05) (drill 1.5) (layers "*.Cu" "*.Mask") (remove_unused_layers no) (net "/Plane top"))
  (pad "2" thru_hole circle (at -2.54 -2.54) (size 2.25 2.25) (drill 1.7) (layers "*.Cu" "*.Mask") (remove_unused_layers no)
   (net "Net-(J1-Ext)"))
  (pad "2" thru_hole circle (at -2.54 2.54) (size 2.25 2.25) (drill 1.7) (layers "*.Cu" "*.Mask") (remove_unused_layers no)
   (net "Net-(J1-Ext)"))
  (pad "2" thru_hole circle (at 2.54 -2.54) (size 2.25 2.25) (drill 1.7) (layers "*.Cu" "*.Mask") (remove_unused_layers no)
   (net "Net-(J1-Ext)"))
  (pad "2" thru_hole circle (at 2.54 2.54) (size 2.25 2.25) (drill 1.7) (layers "*.Cu" "*.Mask") (remove_unused_layers no)
   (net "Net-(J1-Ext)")))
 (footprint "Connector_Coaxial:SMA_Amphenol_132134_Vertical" (layer "F.Cu") (at 105 123.16)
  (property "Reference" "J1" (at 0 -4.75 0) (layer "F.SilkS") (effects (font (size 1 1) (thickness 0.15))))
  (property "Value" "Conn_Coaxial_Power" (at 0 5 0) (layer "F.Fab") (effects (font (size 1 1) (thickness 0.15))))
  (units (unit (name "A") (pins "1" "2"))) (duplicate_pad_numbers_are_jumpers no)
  (pad "1" thru_hole circle (at 0 0) (size 2.05 2.05) (drill 1.5) (layers "*.Cu" "*.Mask") (remove_unused_layers no) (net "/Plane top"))
  (pad "2" thru_hole circle (at -2.54 -2.54) (size 2.25 2.25) (drill 1.7) (layers "*.Cu" "*.Mask") (remove_unused_layers no)
   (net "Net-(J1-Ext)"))
  (pad "2" thru_hole circle (at -2.54 2.54) (size 2.25 2.25) (drill 1.7) (layers "*.Cu" "*.Mask") (remove_unused_layers no)
   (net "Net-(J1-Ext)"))
  (pad "2" thru_hole circle (at 2.54 -2.54) (size 2.25 2.25) (drill 1.7) (layers "*.Cu" "*.Mask") (remove_unused_layers no)
   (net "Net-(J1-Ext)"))
  (pad "2" thru_hole circle (at 2.54 2.54) (size 2.25 2.25) (drill 1.7) (layers "*.Cu" "*.Mask") (remove_unused_layers no)
   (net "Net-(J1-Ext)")))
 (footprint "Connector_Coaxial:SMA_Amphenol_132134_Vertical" (layer "F.Cu") (at 285 123.3)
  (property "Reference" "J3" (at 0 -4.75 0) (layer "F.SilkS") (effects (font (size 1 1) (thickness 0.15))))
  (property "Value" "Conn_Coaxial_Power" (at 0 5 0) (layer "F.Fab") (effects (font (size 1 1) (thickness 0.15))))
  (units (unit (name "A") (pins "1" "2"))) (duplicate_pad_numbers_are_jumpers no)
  (pad "1" thru_hole circle (at 0 0) (size 2.05 2.05) (drill 1.5) (layers "*.Cu" "*.Mask") (remove_unused_layers no) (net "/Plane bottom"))
  (pad "2" thru_hole circle (at -2.54 -2.54) (size 2.25 2.25) (drill 1.7) (layers "*.Cu" "*.Mask") (remove_unused_layers no) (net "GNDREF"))
  (pad "2" thru_hole circle (at -2.54 2.54) (size 2.25 2.25) (drill 1.7) (layers "*.Cu" "*.Mask") (remove_unused_layers no) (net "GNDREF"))
  (pad "2" thru_hole circle (at 2.54 -2.54) (size 2.25 2.25) (drill 1.7) (layers "*.Cu" "*.Mask") (remove_unused_layers no) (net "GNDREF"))
  (pad "2" thru_hole circle (at 2.54 2.54) (size 2.25 2.25) (drill 1.7) (layers "*.Cu" "*.Mask") (remove_unused_layers no) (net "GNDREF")))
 (gr_line (start 95 30) (end 95 230) (stroke (width 0.05) (type default)) (layer "Edge.Cuts"))
 (gr_line (start 95 230) (end 295 230) (stroke (width 0.05) (type default)) (layer "Edge.Cuts"))
 (gr_line (start 295 30) (end 95 30) (stroke (width 0.05) (type default)) (layer "Edge.Cuts"))
 (gr_line (start 295 230) (end 295 30) (stroke (width 0.05) (type default)) (layer "Edge.Cuts"))
 (segment (start 270 130) (end 276.73 136.73) (width 1) (layer "B.Cu") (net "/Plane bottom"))
 (segment (start 276.7 123.3) (end 270 130) (width 1) (layer "B.Cu") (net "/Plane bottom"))
 (segment (start 285 123.3) (end 276.7 123.3) (width 1) (layer "B.Cu") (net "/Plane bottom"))
 (segment (start 270 130) (end 245 130) (width 1) (layer "B.Cu") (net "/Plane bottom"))
 (segment (start 276.73 136.73) (end 285 136.73) (width 1) (layer "B.Cu") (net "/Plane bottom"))
 (segment (start 113.42 136.58) (end 120 130) (width 1) (layer "F.Cu") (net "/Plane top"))
 (segment (start 105 136.58) (end 113.42 136.58) (width 1) (layer "F.Cu") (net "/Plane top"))
 (segment (start 120 130) (end 145 130) (width 1) (layer "F.Cu") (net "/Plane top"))
 (segment (start 105 123.16) (end 113.16 123.16) (width 1) (layer "F.Cu") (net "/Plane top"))
 (segment (start 113.16 123.16) (end 120 130) (width 1) (layer "F.Cu") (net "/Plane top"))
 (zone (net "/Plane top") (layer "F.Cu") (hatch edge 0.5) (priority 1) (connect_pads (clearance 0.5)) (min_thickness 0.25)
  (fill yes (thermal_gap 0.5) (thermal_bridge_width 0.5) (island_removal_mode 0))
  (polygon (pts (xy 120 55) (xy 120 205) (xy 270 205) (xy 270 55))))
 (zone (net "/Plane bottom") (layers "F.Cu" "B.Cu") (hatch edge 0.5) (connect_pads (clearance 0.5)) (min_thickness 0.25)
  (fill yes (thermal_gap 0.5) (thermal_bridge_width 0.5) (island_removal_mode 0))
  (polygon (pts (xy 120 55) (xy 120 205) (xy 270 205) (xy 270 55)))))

